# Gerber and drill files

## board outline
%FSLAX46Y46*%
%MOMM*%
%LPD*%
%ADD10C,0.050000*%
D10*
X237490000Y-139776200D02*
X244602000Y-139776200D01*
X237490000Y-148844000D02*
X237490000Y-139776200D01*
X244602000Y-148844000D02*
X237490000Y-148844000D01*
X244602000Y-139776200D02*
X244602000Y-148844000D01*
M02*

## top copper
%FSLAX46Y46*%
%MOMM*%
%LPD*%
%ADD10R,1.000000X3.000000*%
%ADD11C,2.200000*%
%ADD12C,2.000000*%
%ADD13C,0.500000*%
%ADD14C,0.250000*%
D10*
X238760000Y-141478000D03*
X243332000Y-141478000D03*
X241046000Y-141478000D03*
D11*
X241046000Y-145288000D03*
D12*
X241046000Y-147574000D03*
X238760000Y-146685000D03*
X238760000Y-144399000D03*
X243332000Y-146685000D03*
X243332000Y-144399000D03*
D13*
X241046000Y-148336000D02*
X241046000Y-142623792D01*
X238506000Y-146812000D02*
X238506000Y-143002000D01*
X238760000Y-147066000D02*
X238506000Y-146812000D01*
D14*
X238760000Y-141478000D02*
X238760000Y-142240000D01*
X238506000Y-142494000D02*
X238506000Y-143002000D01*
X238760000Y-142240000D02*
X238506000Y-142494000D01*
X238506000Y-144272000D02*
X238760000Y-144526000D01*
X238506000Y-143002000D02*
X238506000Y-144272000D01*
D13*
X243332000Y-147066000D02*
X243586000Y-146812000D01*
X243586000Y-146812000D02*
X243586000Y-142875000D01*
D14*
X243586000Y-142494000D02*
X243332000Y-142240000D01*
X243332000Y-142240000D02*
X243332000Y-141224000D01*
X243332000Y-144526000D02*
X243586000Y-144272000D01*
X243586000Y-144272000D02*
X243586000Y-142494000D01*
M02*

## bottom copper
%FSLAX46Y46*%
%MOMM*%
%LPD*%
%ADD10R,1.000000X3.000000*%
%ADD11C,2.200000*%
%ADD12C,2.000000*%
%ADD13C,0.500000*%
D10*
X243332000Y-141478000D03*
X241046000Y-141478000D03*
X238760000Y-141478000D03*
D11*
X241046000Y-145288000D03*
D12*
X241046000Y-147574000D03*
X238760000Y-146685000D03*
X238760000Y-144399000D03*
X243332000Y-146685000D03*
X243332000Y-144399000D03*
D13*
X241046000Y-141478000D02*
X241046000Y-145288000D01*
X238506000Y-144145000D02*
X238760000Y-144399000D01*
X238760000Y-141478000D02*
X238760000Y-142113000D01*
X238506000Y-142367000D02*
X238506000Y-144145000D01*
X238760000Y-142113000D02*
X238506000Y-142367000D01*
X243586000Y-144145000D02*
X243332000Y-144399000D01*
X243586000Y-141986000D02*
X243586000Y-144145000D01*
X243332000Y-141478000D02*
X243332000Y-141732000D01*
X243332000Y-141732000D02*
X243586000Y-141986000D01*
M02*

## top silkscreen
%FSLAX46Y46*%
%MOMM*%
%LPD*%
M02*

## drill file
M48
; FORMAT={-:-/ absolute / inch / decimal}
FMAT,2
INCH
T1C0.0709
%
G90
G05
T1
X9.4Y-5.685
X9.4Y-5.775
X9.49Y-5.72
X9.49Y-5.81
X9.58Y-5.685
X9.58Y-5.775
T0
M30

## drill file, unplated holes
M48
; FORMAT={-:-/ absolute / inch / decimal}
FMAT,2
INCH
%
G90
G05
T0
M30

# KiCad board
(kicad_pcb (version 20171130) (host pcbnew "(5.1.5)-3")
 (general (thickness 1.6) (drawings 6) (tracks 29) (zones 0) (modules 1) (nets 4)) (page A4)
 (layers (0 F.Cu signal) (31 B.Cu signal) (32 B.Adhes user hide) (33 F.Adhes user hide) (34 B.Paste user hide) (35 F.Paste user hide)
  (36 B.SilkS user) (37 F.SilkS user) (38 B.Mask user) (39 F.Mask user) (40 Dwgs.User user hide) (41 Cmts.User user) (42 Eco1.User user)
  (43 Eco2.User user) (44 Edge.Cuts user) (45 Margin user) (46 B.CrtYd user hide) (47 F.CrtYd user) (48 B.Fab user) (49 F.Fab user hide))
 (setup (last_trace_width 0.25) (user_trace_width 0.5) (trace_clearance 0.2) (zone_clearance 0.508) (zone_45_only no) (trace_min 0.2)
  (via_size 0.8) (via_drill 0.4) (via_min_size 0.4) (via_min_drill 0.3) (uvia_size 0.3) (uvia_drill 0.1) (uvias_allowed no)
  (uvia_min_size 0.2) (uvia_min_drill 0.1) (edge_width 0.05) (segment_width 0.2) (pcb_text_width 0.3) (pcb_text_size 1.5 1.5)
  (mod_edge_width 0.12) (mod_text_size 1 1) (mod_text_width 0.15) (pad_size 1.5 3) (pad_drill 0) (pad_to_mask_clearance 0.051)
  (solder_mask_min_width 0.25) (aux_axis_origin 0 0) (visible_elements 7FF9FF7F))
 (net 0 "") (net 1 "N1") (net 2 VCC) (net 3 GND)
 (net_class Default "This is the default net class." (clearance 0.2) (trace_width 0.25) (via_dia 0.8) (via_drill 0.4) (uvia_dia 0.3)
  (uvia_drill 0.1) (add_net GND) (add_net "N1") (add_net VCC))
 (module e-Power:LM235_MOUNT (layer F.Cu) (at 241.046 141.478)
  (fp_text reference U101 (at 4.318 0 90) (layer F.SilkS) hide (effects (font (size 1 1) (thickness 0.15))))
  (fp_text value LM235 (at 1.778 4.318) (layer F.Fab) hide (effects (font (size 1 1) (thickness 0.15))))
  (pad 1 smd rect (at 2.286 0) (size 1 3) (layers B.Cu B.Paste B.Mask) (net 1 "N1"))
  (pad 2 smd rect (at 0 0) (size 1 3) (layers B.Cu B.Paste B.Mask) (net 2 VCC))
  (pad 3 smd rect (at -2.286 0) (size 1 3) (layers B.Cu B.Paste B.Mask) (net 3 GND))
  (pad 3 smd rect (at -2.286 0) (size 1 3) (layers F.Cu F.Paste F.Mask) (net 3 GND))
  (pad 1 smd rect (at 2.286 0) (size 1 3) (layers F.Cu F.Paste F.Mask) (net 1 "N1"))
  (pad 2 smd rect (at 0 0) (size 1 3) (layers F.Cu F.Paste F.Mask) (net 2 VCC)))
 (gr_line (start 237.49 139.7762) (end 244.602 139.7762) (layer Edge.Cuts) (width 0.05))
 (gr_line (start 237.49 148.844) (end 237.49 139.7762) (layer Edge.Cuts) (width 0.05))
 (gr_line (start 244.602 148.844) (end 237.49 148.844) (layer Edge.Cuts) (width 0.05))
 (gr_line (start 244.602 139.7762) (end 244.602 148.844) (layer Edge.Cuts) (width 0.05))
 (segment (start 241.046 148.336) (end 241.046 142.623792) (width 0.5) (layer F.Cu) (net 2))
 (via (at 241.046 145.288) (size 2.2) (drill 1.8) (layers F.Cu B.Cu) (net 2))
 (via (at 241.046 147.574) (size 2) (drill 1.8) (layers F.Cu B.Cu) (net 2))
 (segment (start 241.046 141.478) (end 241.046 145.288) (width 0.5) (layer B.Cu) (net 2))
 (segment (start 238.506 146.812) (end 238.506 143.002) (width 0.5) (layer F.Cu) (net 3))
 (segment (start 238.76 147.066) (end 238.506 146.812) (width 0.5) (layer F.Cu) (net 3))
 (segment (start 238.76 141.478) (end 238.76 142.24) (width 0.25) (layer F.Cu) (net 3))
 (segment (start 238.506 142.494) (end 238.506 143.002) (width 0.25) (layer F.Cu) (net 3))
 (segment (start 238.76 142.24) (end 238.506 142.494) (width 0.25) (layer F.Cu) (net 3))
 (segment (start 238.506 144.272) (end 238.76 144.526) (width 0.25) (layer F.Cu) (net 3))
 (segment (start 238.506 143.002) (end 238.506 144.272) (width 0.25) (layer F.Cu) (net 3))
 (via (at 238.76 146.685) (size 2) (drill 1.8) (layers F.Cu B.Cu) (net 3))
 (via (at 238.76 144.399) (size 2) (drill 1.8) (layers F.Cu B.Cu) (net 3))
 (segment (start 238.506 144.145) (end 238.76 144.399) (width 0.5) (layer B.Cu) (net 3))
 (segment (start 238.76 141.478) (end 238.76 142.113) (width 0.5) (layer B.Cu) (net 3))
 (segment (start 238.506 142.367) (end 238.506 144.145) (width 0.5) (layer B.Cu) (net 3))
 (segment (start 238.76 142.113) (end 238.506 142.367) (width 0.5) (layer B.Cu) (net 3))
 (segment (start 243.332 147.066) (end 243.586 146.812) (width 0.5) (layer F.Cu) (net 1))
 (segment (start 243.586 146.812) (end 243.586 142.875) (width 0.5) (layer F.Cu) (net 1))
 (segment (start 243.586 142.494) (end 243.332 142.24) (width 0.25) (layer F.Cu) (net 1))
 (segment (start 243.332 142.24) (end 243.332 141.224) (width 0.25) (layer F.Cu) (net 1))
 (segment (start 243.332 144.526) (end 243.586 144.272) (width 0.25) (layer F.Cu) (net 1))
 (segment (start 243.586 144.272) (end 243.586 142.494) (width 0.25) (layer F.Cu) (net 1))
 (via (at 243.332 146.685) (size 2) (drill 1.8) (layers F.Cu B.Cu) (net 1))
 (via (at 243.332 144.399) (size 2) (drill 1.8) (layers F.Cu B.Cu) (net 1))
 (segment (start 243.586 144.145) (end 243.332 144.399) (width 0.5) (layer B.Cu) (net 1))
 (segment (start 243.586 141.986) (end 243.586 144.145) (width 0.5) (layer B.Cu) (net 1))
 (segment (start 243.332 141.478) (end 243.332 141.732) (width 0.5) (layer B.Cu) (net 1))
 (segment (start 243.332 141.732) (end 243.586 141.986) (width 0.5) (layer B.Cu) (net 1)))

